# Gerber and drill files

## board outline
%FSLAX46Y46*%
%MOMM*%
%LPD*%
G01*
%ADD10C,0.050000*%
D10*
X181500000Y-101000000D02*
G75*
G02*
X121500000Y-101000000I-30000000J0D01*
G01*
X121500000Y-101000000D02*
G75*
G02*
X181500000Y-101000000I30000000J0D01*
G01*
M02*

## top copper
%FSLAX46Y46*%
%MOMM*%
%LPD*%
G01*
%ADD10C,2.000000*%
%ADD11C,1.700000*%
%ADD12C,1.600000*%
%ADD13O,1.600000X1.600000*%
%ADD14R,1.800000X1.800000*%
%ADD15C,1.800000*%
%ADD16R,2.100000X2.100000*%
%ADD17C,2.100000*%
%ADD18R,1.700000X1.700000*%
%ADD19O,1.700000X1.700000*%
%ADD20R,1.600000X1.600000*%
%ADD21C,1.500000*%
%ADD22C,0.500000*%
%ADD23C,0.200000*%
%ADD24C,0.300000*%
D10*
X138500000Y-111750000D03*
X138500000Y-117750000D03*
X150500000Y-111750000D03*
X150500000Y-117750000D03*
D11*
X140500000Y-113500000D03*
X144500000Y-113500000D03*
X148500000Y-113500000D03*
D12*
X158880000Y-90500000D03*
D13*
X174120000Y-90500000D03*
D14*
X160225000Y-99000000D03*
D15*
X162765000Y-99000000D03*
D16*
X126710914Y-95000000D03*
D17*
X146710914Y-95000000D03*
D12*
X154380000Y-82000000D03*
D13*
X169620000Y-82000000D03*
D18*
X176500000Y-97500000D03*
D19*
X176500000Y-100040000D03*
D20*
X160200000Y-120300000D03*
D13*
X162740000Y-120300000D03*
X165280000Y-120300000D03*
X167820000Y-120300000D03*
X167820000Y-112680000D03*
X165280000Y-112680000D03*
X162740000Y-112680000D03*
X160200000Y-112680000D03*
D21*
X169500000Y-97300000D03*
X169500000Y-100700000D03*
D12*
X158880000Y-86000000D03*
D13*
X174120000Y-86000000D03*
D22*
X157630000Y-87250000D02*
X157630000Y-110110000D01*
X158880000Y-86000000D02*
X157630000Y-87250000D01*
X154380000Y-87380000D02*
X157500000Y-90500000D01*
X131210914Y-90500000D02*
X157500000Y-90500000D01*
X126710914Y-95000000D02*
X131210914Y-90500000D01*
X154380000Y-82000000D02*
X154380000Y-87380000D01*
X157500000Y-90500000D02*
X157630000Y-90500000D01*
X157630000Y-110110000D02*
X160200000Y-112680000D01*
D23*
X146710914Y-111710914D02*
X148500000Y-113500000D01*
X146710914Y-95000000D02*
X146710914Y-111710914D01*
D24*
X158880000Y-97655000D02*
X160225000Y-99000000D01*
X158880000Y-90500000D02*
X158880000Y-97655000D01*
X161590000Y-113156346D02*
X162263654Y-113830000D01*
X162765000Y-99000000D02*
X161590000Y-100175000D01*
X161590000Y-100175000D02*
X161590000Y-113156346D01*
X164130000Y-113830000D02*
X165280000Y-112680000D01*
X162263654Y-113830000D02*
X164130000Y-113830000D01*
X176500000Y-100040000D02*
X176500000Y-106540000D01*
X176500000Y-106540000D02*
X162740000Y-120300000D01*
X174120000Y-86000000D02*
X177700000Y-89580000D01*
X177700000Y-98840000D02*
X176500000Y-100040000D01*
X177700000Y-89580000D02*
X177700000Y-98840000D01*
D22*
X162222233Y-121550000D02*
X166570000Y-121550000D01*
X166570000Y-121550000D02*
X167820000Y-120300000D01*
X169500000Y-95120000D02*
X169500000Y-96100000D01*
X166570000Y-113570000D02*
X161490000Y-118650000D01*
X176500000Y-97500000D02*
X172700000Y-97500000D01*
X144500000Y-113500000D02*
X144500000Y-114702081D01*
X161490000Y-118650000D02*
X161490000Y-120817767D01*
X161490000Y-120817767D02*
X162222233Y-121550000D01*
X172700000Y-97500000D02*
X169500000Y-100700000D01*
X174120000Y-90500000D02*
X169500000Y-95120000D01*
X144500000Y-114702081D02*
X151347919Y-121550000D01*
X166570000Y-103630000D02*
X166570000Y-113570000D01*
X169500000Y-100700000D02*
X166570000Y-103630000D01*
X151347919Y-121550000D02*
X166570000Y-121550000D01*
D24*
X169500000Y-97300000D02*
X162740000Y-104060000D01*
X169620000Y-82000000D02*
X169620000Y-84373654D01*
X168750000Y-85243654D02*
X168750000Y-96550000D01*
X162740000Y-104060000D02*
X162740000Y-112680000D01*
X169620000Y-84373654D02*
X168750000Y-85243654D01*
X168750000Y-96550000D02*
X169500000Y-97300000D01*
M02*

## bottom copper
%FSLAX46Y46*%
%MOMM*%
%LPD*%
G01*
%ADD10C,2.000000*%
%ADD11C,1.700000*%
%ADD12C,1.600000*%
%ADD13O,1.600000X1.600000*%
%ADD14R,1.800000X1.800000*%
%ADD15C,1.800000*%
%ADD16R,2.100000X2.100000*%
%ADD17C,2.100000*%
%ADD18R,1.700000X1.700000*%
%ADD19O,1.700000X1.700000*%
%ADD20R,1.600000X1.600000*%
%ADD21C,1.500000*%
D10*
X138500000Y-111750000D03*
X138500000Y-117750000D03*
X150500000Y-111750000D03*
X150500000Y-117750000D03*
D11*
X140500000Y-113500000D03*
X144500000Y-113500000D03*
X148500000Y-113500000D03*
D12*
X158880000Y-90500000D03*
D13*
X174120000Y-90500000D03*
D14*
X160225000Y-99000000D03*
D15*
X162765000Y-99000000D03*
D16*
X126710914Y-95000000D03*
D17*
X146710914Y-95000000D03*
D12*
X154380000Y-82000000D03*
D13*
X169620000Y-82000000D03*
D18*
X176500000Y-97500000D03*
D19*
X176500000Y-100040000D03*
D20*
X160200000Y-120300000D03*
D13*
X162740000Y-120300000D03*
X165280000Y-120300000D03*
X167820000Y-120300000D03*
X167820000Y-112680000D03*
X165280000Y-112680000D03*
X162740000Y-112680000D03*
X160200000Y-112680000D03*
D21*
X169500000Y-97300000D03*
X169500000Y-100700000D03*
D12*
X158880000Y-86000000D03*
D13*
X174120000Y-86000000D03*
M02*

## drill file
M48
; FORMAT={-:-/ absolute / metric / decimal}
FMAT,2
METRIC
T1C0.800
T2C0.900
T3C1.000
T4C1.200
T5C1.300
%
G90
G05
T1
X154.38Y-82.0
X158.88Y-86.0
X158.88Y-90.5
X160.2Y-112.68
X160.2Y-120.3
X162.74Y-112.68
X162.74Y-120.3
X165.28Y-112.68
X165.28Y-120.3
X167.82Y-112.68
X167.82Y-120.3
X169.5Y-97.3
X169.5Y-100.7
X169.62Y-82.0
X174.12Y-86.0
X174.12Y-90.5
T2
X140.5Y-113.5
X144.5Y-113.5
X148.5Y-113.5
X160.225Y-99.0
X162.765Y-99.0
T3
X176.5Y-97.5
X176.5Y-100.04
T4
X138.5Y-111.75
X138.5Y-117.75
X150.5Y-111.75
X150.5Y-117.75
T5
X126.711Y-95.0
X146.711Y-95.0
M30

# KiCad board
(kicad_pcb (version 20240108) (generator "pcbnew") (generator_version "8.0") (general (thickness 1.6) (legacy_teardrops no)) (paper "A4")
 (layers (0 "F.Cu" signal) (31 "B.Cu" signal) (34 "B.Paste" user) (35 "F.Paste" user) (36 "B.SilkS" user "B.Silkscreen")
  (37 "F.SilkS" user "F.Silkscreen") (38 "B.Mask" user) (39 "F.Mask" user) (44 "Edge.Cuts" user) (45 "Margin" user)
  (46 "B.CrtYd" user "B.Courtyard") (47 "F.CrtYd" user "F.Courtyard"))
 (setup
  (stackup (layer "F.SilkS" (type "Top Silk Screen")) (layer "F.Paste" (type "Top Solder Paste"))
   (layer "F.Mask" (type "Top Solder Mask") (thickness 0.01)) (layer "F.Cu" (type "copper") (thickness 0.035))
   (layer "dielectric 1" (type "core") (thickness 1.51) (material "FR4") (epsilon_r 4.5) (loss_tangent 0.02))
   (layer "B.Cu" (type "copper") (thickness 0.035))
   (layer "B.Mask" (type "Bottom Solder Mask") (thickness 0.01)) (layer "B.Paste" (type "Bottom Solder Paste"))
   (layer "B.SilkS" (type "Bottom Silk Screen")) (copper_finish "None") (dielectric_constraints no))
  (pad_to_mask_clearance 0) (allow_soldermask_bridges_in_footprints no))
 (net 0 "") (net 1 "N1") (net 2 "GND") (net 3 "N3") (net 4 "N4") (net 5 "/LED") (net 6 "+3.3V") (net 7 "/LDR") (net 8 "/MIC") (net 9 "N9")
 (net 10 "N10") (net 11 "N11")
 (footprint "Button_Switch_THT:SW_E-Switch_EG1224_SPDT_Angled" (layer "F.Cu") (at 140.5 113.5)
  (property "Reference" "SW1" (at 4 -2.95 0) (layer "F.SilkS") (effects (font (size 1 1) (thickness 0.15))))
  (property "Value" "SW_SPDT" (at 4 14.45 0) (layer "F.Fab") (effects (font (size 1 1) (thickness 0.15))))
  (pad "" thru_hole circle (at -2 -1.75) (size 2 2) (drill 1.2) (layers "*.Cu" "*.Mask") (remove_unused_layers no))
  (pad "" thru_hole circle (at -2 4.25) (size 2 2) (drill 1.2) (layers "*.Cu" "*.Mask") (remove_unused_layers no))
  (pad "" thru_hole circle (at 10 -1.75) (size 2 2) (drill 1.2) (layers "*.Cu" "*.Mask") (remove_unused_layers no))
  (pad "" thru_hole circle (at 10 4.25) (size 2 2) (drill 1.2) (layers "*.Cu" "*.Mask") (remove_unused_layers no))
  (pad "1" thru_hole circle (at 0 0) (size 1.7 1.7) (drill 0.9) (layers "*.Cu" "*.Mask") (remove_unused_layers no) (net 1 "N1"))
  (pad "2" thru_hole circle (at 4 0) (size 1.7 1.7) (drill 0.9) (layers "*.Cu" "*.Mask") (remove_unused_layers no) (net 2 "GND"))
  (pad "3" thru_hole circle (at 8 0) (size 1.7 1.7) (drill 0.9) (layers "*.Cu" "*.Mask") (remove_unused_layers no) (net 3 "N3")))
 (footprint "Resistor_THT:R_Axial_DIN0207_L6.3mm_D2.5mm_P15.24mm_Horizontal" (layer "F.Cu") (at 158.88 90.5)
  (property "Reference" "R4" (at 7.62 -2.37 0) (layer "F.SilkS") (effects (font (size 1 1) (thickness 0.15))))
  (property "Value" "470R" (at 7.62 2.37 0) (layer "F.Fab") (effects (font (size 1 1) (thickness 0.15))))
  (pad "1" thru_hole circle (at 0 0) (size 1.6 1.6) (drill 0.8) (layers "*.Cu" "*.Mask") (remove_unused_layers no) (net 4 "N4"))
  (pad "2" thru_hole oval (at 15.24 0) (size 1.6 1.6) (drill 0.8) (layers "*.Cu" "*.Mask") (remove_unused_layers no) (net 2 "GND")))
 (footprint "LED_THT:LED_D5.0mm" (layer "F.Cu") (at 160.225 99)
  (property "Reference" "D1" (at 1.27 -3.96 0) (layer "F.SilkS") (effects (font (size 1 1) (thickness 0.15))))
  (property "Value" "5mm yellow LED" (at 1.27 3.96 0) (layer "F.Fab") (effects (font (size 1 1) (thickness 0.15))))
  (pad "1" thru_hole rect (at 0 0) (size 1.8 1.8) (drill 0.9) (layers "*.Cu" "*.Mask") (remove_unused_layers no) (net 4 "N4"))
  (pad "2" thru_hole circle (at 2.54 0) (size 1.8 1.8) (drill 0.9) (layers "*.Cu" "*.Mask") (remove_unused_layers no) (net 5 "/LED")))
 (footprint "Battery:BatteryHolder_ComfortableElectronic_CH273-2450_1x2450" (layer "F.Cu") (at 126.710914 95)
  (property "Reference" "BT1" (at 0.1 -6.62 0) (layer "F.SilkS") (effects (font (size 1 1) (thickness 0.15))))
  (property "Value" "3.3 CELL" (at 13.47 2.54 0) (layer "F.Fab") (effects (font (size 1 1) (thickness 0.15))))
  (pad "1" thru_hole rect (at 0 0 270) (size 2.1 2.1) (drill 1.3) (layers "*.Cu" "*.Mask") (remove_unused_layers no) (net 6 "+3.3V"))
  (pad "2" thru_hole circle (at 20 0 270) (size 2.1 2.1) (drill 1.3) (layers "*.Cu" "*.Mask") (remove_unused_layers no) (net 3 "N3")))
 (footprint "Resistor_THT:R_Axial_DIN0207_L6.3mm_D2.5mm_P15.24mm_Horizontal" (layer "F.Cu") (at 154.38 82)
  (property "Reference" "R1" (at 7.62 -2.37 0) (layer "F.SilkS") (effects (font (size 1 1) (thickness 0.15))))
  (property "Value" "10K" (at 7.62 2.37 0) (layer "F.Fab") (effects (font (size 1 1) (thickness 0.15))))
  (pad "1" thru_hole circle (at 0 0) (size 1.6 1.6) (drill 0.8) (layers "*.Cu" "*.Mask") (remove_unused_layers no) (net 6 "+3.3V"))
  (pad "2" thru_hole oval (at 15.24 0) (size 1.6 1.6) (drill 0.8) (layers "*.Cu" "*.Mask") (remove_unused_layers no) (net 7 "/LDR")))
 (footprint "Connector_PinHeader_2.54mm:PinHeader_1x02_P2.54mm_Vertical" (layer "F.Cu") (at 176.5 97.5)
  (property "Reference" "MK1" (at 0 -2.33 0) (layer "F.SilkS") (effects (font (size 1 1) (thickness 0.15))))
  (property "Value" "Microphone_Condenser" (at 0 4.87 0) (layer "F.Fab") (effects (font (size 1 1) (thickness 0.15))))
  (pad "1" thru_hole rect (at 0 0) (size 1.7 1.7) (drill 1) (layers "*.Cu" "*.Mask") (remove_unused_layers no) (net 2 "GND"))
  (pad "2" thru_hole oval (at 0 2.54) (size 1.7 1.7) (drill 1) (layers "*.Cu" "*.Mask") (remove_unused_layers no) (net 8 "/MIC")))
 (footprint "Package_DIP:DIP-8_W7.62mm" (layer "F.Cu") (at 160.2 120.3 90)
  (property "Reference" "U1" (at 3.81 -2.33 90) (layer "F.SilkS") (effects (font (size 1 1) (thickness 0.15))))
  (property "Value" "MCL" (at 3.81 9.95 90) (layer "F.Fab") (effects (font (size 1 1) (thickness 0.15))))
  (pad "1" thru_hole rect (at 0 0 90) (size 1.6 1.6) (drill 0.8) (layers "*.Cu" "*.Mask") (remove_unused_layers no) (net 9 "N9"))
  (pad "2" thru_hole oval (at 0 2.54 90) (size 1.6 1.6) (drill 0.8) (layers "*.Cu" "*.Mask") (remove_unused_layers no) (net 8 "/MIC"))
  (pad "3" thru_hole oval (at 0 5.08 90) (size 1.6 1.6) (drill 0.8) (layers "*.Cu" "*.Mask") (remove_unused_layers no) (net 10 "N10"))
  (pad "4" thru_hole oval (at 0 7.62 90) (size 1.6 1.6) (drill 0.8) (layers "*.Cu" "*.Mask") (remove_unused_layers no) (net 2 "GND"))
  (pad "5" thru_hole oval (at 7.62 7.62 90) (size 1.6 1.6) (drill 0.8) (layers "*.Cu" "*.Mask") (remove_unused_layers no) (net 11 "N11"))
  (pad "6" thru_hole oval (at 7.62 5.08 90) (size 1.6 1.6) (drill 0.8) (layers "*.Cu" "*.Mask") (remove_unused_layers no) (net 5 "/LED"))
  (pad "7" thru_hole oval (at 7.62 2.54 90) (size 1.6 1.6) (drill 0.8) (layers "*.Cu" "*.Mask") (remove_unused_layers no) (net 7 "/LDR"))
  (pad "8" thru_hole oval (at 7.62 0 90) (size 1.6 1.6) (drill 0.8) (layers "*.Cu" "*.Mask") (remove_unused_layers no) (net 6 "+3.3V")))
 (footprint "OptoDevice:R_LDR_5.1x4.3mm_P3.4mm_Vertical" (layer "F.Cu") (at 169.5 97.3 -90)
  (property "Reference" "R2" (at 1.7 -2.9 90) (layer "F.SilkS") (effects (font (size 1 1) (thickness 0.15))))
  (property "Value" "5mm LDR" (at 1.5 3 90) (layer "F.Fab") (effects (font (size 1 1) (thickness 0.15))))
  (pad "1" thru_hole circle (at 0 0 270) (size 1.5 1.5) (drill 0.8) (layers "*.Cu" "*.Mask") (remove_unused_layers no) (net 7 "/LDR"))
  (pad "2" thru_hole circle (at 3.4 0 270) (size 1.5 1.5) (drill 0.8) (layers "*.Cu" "*.Mask") (remove_unused_layers no) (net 2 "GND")))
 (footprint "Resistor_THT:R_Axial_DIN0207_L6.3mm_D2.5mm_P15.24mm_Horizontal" (layer "F.Cu") (at 158.88 86)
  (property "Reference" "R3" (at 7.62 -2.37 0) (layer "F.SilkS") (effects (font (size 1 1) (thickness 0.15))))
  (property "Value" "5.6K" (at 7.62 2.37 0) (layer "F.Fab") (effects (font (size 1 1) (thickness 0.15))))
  (pad "1" thru_hole circle (at 0 0) (size 1.6 1.6) (drill 0.8) (layers "*.Cu" "*.Mask") (remove_unused_layers no) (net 6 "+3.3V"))
  (pad "2" thru_hole oval (at 15.24 0) (size 1.6 1.6) (drill 0.8) (layers "*.Cu" "*.Mask") (remove_unused_layers no) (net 8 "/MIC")))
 (gr_circle (center 151.5 101) (end 181.5 101) (locked yes) (stroke (width 0.05) (type default)) (fill none) (layer "Edge.Cuts"))
 (segment (start 157.63 87.25) (end 157.63 110.11) (width 0.5) (layer "F.Cu") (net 6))
 (segment (start 158.88 86) (end 157.63 87.25) (width 0.5) (layer "F.Cu") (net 6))
 (segment (start 154.38 87.38) (end 157.5 90.5) (width 0.5) (layer "F.Cu") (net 6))
 (segment (start 131.210914 90.5) (end 157.5 90.5) (width 0.5) (layer "F.Cu") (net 6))
 (segment (start 126.710914 95) (end 131.210914 90.5) (width 0.5) (layer "F.Cu") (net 6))
 (segment (start 154.38 82) (end 154.38 87.38) (width 0.5) (layer "F.Cu") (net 6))
 (segment (start 157.5 90.5) (end 157.63 90.5) (width 0.5) (layer "F.Cu") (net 6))
 (segment (start 157.63 110.11) (end 160.2 112.68) (width 0.5) (layer "F.Cu") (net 6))
 (segment (start 146.710914 111.710914) (end 148.5 113.5) (width 0.2) (layer "F.Cu") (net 3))
 (segment (start 146.710914 95) (end 146.710914 111.710914) (width 0.2) (layer "F.Cu") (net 3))
 (segment (start 158.88 97.655) (end 160.225 99) (width 0.3) (layer "F.Cu") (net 4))
 (segment (start 158.88 90.5) (end 158.88 97.655) (width 0.3) (layer "F.Cu") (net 4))
 (segment (start 161.59 113.156346) (end 162.263654 113.83) (width 0.3) (layer "F.Cu") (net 5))
 (segment (start 162.765 99) (end 161.59 100.175) (width 0.3) (layer "F.Cu") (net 5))
 (segment (start 161.59 100.175) (end 161.59 113.156346) (width 0.3) (layer "F.Cu") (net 5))
 (segment (start 164.13 113.83) (end 165.28 112.68) (width 0.3) (layer "F.Cu") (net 5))
 (segment (start 162.263654 113.83) (end 164.13 113.83) (width 0.3) (layer "F.Cu") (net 5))
 (segment (start 176.5 100.04) (end 176.5 106.54) (width 0.3) (layer "F.Cu") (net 8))
 (segment (start 176.5 106.54) (end 162.74 120.3) (width 0.3) (layer "F.Cu") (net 8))
 (segment (start 174.12 86) (end 177.7 89.58) (width 0.3) (layer "F.Cu") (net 8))
 (segment (start 177.7 98.84) (end 176.5 100.04) (width 0.3) (layer "F.Cu") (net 8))
 (segment (start 177.7 89.58) (end 177.7 98.84) (width 0.3) (layer "F.Cu") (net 8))
 (segment (start 162.222233 121.55) (end 166.57 121.55) (width 0.5) (layer "F.Cu") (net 2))
 (segment (start 166.57 121.55) (end 167.82 120.3) (width 0.5) (layer "F.Cu") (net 2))
 (segment (start 169.5 95.12) (end 169.5 96.1) (width 0.5) (layer "F.Cu") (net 2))
 (segment (start 166.57 113.57) (end 161.49 118.65) (width 0.5) (layer "F.Cu") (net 2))
 (segment (start 176.5 97.5) (end 172.7 97.5) (width 0.5) (layer "F.Cu") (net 2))
 (segment (start 144.5 113.5) (end 144.5 114.702081) (width 0.5) (layer "F.Cu") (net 2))
 (segment (start 161.49 118.65) (end 161.49 120.817767) (width 0.5) (layer "F.Cu") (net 2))
 (segment (start 161.49 120.817767) (end 162.222233 121.55) (width 0.5) (layer "F.Cu") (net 2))
 (segment (start 172.7 97.5) (end 169.5 100.7) (width 0.5) (layer "F.Cu") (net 2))
 (segment (start 174.12 90.5) (end 169.5 95.12) (width 0.5) (layer "F.Cu") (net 2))
 (segment (start 144.5 114.702081) (end 151.347919 121.55) (width 0.5) (layer "F.Cu") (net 2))
 (segment (start 166.57 103.63) (end 166.57 113.57) (width 0.5) (layer "F.Cu") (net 2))
 (segment (start 169.5 100.7) (end 166.57 103.63) (width 0.5) (layer "F.Cu") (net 2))
 (segment (start 151.347919 121.55) (end 166.57 121.55) (width 0.5) (layer "F.Cu") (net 2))
 (segment (start 169.5 97.3) (end 162.74 104.06) (width 0.3) (layer "F.Cu") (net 7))
 (segment (start 169.62 82) (end 169.62 84.373654) (width 0.3) (layer "F.Cu") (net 7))
 (segment (start 168.75 85.243654) (end 168.75 96.55) (width 0.3) (layer "F.Cu") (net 7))
 (segment (start 162.74 104.06) (end 162.74 112.68) (width 0.3) (layer "F.Cu") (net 7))
 (segment (start 169.62 84.373654) (end 168.75 85.243654) (width 0.3) (layer "F.Cu") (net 7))
 (segment (start 168.75 96.55) (end 169.5 97.3) (width 0.3) (layer "F.Cu") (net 7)))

